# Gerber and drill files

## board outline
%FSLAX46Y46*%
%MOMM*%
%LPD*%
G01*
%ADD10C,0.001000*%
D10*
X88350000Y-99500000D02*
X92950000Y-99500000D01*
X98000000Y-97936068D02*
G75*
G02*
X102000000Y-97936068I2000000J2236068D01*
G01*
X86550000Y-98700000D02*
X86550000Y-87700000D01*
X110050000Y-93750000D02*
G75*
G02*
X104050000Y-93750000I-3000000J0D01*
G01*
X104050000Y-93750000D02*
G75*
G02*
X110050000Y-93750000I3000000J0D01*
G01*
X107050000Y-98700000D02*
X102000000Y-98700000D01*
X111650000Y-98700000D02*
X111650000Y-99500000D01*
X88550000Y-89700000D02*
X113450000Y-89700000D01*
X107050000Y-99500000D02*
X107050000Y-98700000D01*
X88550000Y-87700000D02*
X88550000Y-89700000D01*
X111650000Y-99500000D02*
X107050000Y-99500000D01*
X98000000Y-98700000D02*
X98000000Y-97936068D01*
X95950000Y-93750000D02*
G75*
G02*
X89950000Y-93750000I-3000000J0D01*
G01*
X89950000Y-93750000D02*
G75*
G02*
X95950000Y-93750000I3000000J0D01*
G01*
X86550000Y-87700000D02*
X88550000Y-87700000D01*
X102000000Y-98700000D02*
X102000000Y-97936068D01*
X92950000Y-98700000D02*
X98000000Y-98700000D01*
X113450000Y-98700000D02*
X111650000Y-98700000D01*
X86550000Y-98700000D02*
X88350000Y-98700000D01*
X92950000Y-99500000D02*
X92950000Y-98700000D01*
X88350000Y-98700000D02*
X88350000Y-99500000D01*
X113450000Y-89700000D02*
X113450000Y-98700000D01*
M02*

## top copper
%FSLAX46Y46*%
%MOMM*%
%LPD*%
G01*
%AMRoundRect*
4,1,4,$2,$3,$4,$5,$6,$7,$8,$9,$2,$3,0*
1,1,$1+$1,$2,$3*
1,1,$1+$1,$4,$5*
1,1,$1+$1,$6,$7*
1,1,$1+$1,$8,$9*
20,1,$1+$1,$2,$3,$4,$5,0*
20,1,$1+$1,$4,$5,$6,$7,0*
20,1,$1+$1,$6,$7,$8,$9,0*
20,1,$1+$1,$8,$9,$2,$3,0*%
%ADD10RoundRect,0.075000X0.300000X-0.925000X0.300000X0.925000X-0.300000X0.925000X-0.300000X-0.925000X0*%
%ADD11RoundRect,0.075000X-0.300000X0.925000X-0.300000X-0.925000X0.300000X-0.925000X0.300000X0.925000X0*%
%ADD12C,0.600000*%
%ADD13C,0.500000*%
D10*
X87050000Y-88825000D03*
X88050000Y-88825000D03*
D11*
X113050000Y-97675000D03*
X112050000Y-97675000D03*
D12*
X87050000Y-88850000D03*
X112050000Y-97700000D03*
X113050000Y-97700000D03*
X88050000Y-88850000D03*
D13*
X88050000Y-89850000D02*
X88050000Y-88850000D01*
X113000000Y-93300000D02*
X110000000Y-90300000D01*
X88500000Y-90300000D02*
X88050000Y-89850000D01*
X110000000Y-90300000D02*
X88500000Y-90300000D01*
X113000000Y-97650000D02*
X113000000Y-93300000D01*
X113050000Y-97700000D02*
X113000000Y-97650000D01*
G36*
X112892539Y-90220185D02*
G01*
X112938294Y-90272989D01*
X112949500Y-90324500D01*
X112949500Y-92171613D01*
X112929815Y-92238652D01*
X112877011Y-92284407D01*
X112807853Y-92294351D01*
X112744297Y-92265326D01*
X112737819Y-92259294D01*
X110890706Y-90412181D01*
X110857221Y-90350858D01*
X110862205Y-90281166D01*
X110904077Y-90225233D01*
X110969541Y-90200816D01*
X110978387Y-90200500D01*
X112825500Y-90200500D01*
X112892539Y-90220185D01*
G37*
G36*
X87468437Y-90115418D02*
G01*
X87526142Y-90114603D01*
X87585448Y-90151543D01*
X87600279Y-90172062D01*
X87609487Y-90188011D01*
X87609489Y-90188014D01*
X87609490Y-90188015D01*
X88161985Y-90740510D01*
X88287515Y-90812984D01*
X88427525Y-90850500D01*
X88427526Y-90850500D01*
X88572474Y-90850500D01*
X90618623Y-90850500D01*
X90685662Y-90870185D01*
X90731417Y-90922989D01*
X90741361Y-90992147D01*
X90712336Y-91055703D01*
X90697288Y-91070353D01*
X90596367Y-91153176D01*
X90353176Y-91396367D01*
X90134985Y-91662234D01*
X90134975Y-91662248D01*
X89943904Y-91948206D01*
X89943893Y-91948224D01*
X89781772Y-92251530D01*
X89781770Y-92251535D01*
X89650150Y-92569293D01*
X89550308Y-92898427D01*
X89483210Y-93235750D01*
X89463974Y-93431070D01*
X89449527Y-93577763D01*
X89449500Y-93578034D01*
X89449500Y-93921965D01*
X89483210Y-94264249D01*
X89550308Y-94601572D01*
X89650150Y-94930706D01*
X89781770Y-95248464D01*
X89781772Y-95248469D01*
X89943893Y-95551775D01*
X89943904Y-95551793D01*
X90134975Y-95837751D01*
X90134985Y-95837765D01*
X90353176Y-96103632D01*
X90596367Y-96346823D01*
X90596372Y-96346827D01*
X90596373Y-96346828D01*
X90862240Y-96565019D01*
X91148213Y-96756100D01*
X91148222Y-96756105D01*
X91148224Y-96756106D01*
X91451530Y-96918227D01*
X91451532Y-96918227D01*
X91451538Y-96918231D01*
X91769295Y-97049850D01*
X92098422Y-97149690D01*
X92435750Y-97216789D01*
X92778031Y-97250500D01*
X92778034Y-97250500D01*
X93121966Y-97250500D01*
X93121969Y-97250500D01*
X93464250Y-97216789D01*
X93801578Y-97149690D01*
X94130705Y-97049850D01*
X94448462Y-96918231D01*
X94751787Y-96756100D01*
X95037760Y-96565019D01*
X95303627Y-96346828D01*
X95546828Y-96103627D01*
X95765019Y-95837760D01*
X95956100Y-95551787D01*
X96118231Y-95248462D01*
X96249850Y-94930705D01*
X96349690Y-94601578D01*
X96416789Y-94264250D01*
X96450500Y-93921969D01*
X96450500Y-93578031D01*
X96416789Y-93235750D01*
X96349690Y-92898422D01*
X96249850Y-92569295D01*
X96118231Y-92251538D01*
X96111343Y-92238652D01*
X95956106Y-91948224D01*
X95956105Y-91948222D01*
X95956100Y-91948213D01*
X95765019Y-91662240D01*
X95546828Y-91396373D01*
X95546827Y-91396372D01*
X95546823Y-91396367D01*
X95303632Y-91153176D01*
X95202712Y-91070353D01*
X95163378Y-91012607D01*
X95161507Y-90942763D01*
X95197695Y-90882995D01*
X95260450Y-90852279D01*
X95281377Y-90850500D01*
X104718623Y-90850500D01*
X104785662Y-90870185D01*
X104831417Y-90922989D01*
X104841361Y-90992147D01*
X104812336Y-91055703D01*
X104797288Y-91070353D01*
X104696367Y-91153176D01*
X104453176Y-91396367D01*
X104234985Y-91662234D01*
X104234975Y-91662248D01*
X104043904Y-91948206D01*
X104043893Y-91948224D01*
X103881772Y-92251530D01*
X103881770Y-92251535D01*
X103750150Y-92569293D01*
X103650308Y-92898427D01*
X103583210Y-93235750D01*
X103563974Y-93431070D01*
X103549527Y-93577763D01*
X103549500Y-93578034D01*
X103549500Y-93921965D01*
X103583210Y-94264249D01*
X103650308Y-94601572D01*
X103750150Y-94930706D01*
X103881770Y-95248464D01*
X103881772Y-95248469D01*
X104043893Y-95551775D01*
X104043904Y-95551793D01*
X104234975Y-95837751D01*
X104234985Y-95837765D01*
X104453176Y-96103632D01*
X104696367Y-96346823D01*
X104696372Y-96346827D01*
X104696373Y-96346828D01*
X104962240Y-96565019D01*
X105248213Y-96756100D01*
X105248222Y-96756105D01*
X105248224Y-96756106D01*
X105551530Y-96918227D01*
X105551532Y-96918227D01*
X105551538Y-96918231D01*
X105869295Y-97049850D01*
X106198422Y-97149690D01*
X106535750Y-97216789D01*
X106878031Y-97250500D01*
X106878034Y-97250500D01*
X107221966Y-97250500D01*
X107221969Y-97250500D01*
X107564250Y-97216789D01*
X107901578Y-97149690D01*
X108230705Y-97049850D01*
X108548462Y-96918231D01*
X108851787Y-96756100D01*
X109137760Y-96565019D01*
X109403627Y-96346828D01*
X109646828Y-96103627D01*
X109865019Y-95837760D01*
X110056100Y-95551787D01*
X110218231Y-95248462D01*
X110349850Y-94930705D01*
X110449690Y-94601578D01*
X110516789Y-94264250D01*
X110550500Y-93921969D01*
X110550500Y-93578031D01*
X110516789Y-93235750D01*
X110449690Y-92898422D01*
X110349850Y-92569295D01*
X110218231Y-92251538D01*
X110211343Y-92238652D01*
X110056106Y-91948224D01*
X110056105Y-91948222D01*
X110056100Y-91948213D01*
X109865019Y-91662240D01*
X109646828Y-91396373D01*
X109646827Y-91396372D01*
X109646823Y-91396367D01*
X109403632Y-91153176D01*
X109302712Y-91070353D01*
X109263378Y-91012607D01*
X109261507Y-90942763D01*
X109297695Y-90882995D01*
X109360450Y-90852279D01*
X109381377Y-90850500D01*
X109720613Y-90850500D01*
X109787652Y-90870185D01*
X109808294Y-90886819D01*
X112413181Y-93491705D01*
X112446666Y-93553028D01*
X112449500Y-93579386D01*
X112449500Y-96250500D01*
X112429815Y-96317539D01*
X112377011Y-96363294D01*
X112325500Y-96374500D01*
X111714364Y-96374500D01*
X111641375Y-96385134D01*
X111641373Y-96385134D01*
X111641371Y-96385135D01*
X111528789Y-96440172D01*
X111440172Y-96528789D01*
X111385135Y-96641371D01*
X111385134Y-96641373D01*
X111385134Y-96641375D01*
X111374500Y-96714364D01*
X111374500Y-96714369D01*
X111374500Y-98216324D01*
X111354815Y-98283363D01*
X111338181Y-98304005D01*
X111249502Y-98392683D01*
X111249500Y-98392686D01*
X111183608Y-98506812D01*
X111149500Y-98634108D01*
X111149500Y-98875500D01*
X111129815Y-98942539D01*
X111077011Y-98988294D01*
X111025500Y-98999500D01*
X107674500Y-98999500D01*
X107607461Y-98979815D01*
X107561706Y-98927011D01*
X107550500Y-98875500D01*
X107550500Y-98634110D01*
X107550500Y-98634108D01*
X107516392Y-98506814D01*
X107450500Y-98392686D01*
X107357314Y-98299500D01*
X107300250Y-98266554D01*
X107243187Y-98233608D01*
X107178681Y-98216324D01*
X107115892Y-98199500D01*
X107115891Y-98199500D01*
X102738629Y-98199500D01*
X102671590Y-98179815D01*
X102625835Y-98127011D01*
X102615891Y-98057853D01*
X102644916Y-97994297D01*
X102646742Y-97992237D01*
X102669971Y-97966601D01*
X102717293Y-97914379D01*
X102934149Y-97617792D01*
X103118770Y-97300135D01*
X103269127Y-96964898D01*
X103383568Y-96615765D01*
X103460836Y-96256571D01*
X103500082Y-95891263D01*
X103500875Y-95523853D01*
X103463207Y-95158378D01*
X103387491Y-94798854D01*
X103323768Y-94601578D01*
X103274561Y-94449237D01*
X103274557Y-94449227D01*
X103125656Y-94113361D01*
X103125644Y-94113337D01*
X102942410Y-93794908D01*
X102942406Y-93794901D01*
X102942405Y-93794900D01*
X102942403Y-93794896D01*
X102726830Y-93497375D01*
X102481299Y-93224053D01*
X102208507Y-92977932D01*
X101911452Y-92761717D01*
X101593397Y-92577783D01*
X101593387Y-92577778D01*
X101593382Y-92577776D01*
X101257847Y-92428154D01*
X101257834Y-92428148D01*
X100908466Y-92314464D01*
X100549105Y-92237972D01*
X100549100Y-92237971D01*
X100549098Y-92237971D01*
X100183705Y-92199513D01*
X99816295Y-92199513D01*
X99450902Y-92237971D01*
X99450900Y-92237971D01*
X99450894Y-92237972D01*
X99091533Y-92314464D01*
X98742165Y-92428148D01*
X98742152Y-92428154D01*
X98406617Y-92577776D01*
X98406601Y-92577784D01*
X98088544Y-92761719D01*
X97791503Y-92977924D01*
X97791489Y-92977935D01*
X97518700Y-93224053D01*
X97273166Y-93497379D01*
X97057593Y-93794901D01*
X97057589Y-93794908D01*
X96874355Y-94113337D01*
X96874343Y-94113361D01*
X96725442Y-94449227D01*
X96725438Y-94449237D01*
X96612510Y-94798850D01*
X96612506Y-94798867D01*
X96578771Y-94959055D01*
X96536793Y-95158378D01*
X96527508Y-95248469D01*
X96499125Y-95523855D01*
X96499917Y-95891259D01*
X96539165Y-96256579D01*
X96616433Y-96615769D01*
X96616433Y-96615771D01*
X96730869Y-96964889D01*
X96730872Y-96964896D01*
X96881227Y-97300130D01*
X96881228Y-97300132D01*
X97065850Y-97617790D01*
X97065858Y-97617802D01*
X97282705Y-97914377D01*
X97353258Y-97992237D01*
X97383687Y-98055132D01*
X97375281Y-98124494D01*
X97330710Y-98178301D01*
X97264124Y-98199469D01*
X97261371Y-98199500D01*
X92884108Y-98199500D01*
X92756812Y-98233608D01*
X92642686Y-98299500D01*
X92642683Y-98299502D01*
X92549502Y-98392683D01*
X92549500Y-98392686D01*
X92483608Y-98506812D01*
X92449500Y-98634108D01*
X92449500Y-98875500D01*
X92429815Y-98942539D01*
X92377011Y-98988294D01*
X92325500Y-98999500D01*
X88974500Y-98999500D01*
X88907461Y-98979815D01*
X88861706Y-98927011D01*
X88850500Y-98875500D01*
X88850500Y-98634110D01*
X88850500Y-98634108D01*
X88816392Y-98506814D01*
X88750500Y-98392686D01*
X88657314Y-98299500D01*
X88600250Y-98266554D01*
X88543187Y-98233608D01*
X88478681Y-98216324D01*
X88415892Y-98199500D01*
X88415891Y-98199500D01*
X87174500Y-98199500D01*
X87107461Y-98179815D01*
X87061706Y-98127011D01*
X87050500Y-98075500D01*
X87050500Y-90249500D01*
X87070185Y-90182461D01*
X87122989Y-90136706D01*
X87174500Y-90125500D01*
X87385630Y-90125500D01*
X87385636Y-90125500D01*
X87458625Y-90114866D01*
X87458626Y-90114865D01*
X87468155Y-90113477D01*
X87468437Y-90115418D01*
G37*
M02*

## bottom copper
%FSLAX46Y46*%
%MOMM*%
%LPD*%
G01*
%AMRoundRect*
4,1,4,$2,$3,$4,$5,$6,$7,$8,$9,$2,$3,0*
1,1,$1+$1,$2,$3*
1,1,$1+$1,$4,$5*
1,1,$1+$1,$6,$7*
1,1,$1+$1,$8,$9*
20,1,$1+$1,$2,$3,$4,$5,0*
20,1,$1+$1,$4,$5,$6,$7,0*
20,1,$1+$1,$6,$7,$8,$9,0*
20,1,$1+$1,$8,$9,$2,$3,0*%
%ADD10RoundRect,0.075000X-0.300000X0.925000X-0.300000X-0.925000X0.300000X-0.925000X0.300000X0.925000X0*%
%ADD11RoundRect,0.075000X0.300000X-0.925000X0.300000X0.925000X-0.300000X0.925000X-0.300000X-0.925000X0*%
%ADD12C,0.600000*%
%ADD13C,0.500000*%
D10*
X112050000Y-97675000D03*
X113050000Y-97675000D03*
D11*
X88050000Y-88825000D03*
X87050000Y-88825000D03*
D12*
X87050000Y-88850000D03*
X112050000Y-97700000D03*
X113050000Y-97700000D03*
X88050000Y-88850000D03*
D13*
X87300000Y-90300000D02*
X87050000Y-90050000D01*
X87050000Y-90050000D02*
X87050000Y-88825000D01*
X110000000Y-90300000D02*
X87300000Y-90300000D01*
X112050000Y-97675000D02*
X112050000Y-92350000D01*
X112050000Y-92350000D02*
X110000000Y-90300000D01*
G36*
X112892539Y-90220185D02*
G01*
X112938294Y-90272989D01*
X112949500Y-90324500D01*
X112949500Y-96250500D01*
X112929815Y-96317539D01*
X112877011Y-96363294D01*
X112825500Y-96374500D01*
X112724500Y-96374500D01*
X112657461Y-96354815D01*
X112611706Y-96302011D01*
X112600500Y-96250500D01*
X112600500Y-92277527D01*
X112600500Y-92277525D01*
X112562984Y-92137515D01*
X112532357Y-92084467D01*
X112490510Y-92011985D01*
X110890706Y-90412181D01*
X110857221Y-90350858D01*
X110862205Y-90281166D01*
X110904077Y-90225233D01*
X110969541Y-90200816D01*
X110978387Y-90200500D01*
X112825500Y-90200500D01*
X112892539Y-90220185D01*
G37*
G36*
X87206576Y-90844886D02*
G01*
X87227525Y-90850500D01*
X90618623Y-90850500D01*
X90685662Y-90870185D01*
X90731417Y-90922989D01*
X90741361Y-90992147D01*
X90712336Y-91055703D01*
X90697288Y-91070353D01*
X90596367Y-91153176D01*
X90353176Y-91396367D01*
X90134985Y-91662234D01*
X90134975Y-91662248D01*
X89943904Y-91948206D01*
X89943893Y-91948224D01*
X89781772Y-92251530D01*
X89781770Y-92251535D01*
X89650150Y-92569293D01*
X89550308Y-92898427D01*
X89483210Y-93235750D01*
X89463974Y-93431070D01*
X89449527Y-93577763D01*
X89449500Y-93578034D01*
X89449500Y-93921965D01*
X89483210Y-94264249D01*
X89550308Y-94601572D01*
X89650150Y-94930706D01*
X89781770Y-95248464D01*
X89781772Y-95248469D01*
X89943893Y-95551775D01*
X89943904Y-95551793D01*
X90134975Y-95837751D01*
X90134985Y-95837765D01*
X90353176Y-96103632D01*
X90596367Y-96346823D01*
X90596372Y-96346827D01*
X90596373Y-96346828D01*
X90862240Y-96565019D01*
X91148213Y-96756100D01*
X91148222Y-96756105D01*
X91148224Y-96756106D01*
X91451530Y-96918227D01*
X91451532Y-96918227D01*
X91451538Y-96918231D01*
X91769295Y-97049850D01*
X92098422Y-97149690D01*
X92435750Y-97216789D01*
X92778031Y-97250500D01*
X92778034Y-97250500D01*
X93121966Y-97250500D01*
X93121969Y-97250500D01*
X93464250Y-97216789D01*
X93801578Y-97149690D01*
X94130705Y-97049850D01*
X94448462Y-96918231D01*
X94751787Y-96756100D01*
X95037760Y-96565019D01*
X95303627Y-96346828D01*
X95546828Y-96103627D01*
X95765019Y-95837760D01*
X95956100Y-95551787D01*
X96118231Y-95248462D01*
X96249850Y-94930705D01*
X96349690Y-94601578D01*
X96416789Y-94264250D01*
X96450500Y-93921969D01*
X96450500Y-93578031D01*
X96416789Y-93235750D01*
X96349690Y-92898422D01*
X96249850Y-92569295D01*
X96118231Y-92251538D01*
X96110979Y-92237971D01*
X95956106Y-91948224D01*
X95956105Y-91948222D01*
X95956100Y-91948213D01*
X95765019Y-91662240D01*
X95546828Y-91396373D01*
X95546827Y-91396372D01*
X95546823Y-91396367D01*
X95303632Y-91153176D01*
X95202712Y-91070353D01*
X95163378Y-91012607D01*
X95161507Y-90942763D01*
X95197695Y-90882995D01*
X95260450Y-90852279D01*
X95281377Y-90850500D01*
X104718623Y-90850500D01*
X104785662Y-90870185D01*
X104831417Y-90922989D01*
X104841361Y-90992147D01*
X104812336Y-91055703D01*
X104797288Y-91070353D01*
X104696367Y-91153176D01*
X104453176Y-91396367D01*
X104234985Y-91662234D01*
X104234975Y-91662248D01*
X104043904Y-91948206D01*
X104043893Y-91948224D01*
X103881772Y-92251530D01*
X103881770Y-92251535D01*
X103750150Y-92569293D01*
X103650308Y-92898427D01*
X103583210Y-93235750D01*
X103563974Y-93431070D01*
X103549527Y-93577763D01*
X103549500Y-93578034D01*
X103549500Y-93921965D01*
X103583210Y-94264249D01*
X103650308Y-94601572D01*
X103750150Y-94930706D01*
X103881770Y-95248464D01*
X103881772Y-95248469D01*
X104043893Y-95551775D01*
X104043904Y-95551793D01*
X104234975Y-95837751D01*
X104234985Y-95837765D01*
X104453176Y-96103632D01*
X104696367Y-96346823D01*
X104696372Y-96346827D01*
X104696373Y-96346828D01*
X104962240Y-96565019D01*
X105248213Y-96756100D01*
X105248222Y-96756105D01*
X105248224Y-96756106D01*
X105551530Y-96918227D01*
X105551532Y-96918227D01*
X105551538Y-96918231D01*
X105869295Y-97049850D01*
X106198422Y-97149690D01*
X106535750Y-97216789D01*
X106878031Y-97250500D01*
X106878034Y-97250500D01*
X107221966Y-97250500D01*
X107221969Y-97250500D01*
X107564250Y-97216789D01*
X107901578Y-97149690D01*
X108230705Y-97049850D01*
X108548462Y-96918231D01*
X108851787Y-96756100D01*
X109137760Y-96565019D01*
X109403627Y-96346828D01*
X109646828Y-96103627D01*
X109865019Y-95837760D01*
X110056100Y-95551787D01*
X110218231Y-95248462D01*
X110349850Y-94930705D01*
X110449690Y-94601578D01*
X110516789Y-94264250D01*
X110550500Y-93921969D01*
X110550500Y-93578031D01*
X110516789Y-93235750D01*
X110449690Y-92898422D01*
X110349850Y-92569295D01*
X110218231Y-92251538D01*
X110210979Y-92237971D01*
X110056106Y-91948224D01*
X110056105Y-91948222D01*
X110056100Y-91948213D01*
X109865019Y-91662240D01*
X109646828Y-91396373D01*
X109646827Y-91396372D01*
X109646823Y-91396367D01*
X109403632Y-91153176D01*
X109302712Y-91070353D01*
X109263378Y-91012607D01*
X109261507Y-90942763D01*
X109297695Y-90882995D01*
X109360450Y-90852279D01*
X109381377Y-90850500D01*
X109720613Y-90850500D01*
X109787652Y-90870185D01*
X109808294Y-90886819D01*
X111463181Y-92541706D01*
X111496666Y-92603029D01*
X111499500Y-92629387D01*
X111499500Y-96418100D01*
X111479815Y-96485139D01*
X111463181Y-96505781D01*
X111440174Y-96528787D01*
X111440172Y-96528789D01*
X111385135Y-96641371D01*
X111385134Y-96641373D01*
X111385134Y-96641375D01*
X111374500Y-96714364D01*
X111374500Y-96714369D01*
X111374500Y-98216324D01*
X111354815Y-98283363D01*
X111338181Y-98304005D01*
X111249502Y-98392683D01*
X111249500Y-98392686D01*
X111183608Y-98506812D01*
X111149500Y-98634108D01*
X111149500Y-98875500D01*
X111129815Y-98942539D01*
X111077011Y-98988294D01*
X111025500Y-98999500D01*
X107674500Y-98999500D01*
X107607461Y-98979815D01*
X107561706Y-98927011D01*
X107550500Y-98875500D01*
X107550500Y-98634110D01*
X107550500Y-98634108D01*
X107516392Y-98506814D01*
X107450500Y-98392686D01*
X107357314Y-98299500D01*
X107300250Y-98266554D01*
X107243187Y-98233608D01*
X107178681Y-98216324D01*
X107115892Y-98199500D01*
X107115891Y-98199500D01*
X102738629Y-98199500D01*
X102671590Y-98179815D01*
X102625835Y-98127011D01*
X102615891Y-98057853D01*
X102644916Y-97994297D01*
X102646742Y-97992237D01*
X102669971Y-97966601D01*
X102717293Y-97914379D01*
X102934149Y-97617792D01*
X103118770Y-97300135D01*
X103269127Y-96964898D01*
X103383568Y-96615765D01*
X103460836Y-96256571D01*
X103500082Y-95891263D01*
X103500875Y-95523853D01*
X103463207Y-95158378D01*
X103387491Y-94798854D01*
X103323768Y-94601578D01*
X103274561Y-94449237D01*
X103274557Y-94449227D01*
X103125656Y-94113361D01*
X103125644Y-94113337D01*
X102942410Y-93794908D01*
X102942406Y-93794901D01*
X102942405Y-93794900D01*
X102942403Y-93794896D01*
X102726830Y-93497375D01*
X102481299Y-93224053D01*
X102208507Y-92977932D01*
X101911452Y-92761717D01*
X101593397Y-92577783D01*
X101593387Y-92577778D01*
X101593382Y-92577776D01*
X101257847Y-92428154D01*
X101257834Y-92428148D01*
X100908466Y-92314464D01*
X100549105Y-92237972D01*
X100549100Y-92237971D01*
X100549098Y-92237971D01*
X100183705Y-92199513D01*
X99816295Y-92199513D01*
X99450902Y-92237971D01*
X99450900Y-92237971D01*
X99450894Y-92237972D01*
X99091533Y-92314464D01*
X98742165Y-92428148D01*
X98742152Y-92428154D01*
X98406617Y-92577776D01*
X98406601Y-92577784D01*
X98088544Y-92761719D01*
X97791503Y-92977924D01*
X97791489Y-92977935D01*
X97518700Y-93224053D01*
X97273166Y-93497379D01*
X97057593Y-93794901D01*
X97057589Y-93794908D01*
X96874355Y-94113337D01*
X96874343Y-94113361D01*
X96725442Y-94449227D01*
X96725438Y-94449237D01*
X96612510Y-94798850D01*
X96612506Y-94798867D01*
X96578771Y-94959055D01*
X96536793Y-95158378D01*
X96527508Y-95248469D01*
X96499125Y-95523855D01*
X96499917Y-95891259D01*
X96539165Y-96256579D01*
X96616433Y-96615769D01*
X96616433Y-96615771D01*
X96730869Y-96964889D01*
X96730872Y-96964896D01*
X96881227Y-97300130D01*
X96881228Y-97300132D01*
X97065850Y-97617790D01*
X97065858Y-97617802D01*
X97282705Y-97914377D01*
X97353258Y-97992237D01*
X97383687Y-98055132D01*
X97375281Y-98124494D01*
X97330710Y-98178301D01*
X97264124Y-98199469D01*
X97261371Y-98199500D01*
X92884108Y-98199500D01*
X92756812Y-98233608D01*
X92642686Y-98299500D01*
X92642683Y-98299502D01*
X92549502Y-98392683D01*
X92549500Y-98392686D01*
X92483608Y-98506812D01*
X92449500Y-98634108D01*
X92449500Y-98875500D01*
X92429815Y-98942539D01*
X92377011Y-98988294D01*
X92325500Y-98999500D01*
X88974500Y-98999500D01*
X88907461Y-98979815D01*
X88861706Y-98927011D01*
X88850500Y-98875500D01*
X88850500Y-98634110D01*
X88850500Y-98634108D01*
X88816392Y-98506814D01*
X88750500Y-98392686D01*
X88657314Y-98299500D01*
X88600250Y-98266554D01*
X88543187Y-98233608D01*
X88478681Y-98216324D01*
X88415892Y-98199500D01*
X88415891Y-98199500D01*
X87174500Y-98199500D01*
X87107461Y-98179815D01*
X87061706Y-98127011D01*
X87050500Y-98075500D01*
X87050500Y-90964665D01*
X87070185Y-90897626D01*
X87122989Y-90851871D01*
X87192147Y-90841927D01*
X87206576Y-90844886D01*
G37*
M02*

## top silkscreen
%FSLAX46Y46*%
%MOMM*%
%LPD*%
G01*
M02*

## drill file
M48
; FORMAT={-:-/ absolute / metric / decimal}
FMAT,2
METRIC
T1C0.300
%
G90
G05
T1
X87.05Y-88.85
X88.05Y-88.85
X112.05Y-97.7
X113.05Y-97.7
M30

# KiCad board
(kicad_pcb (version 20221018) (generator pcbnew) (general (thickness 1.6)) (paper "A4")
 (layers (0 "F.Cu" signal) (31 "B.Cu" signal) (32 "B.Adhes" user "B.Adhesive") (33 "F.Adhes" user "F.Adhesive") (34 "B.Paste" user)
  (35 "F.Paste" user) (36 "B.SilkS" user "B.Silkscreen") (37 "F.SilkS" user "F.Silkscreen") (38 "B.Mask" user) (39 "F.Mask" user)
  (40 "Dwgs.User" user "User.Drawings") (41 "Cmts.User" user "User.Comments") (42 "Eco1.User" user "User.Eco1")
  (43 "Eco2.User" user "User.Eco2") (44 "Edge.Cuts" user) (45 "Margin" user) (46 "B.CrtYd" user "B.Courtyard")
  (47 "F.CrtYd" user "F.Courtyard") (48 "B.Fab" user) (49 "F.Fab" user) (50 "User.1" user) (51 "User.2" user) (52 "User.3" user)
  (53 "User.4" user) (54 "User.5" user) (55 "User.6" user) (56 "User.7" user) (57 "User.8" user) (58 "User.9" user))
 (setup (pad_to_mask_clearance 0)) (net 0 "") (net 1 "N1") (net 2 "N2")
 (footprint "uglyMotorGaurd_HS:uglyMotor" (layer "F.Cu") (at 87.55 89.825)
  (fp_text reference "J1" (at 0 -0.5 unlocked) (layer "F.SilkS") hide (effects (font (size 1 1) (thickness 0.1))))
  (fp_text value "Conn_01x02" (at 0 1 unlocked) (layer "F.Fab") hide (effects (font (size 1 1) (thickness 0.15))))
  (pad "1" smd roundrect (at -0.5 -1 90) (size 2 0.75) (layers "F.Cu" "F.Paste" "F.Mask") (roundrect_rratio 0.1) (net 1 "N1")
   (thermal_bridge_angle 45))
  (pad "2" smd roundrect (at 0.5 -1 90) (size 2 0.75) (layers "F.Cu" "F.Paste" "F.Mask") (roundrect_rratio 0.1) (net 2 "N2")
   (thermal_bridge_angle 45)))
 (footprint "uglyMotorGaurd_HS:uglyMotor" (layer "F.Cu") (at 112.55 96.675 180)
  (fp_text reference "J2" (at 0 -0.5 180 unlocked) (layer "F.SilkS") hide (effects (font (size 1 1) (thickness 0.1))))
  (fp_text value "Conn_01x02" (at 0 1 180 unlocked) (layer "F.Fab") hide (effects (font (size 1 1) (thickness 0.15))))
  (pad "1" smd roundrect (at -0.5 -1 270) (size 2 0.75) (layers "F.Cu" "F.Paste" "F.Mask") (roundrect_rratio 0.1) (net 2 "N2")
   (thermal_bridge_angle 45))
  (pad "2" smd roundrect (at 0.5 -1 270) (size 2 0.75) (layers "F.Cu" "F.Paste" "F.Mask") (roundrect_rratio 0.1) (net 1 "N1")
   (thermal_bridge_angle 45)))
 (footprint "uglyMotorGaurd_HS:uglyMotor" (layer "B.Cu") (at 112.55 96.675)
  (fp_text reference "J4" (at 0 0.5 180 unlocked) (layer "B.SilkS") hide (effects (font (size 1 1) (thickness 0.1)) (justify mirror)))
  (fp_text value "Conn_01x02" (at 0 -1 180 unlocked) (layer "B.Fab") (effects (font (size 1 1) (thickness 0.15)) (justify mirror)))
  (pad "1" smd roundrect (at -0.5 1 270) (size 2 0.75) (layers "B.Cu" "B.Paste" "B.Mask") (roundrect_rratio 0.1) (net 1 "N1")
   (thermal_bridge_angle 45))
  (pad "2" smd roundrect (at 0.5 1 270) (size 2 0.75) (layers "B.Cu" "B.Paste" "B.Mask") (roundrect_rratio 0.1) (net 2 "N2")
   (thermal_bridge_angle 45)))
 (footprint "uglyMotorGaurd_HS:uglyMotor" (layer "B.Cu") (at 87.55 89.825 180)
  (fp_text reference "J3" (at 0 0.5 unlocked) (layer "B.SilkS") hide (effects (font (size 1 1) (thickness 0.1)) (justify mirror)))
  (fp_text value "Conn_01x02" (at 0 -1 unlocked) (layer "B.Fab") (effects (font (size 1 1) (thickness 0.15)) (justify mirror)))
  (pad "1" smd roundrect (at -0.5 1 90) (size 2 0.75) (layers "B.Cu" "B.Paste" "B.Mask") (roundrect_rratio 0.1) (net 2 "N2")
   (thermal_bridge_angle 45))
  (pad "2" smd roundrect (at 0.5 1 90) (size 2 0.75) (layers "B.Cu" "B.Paste" "B.Mask") (roundrect_rratio 0.1) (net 1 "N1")
   (thermal_bridge_angle 45)))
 (gr_line (start 88.35 99.5) (end 92.95 99.5) (stroke (width 0.001) (type solid)) (layer "Edge.Cuts"))
 (gr_arc (start 98 97.936068) (mid 100 92.7) (end 102 97.936068) (stroke (width 0.001) (type solid)) (layer "Edge.Cuts"))
 (gr_line (start 86.55 98.7) (end 86.55 87.7) (stroke (width 0.001) (type solid)) (layer "Edge.Cuts"))
 (gr_circle (center 107.05 93.75) (end 110.05 93.75) (stroke (width 0.001) (type solid)) (fill none) (layer "Edge.Cuts"))
 (gr_line (start 107.05 98.7) (end 102 98.7) (stroke (width 0.001) (type solid)) (layer "Edge.Cuts"))
 (gr_line (start 111.65 98.7) (end 111.65 99.5) (stroke (width 0.001) (type solid)) (layer "Edge.Cuts"))
 (gr_line (start 88.55 89.7) (end 113.45 89.7) (stroke (width 0.001) (type solid)) (layer "Edge.Cuts"))
 (gr_line (start 107.05 99.5) (end 107.05 98.7) (stroke (width 0.001) (type solid)) (layer "Edge.Cuts"))
 (gr_line (start 88.55 87.7) (end 88.55 89.7) (stroke (width 0.001) (type solid)) (layer "Edge.Cuts"))
 (gr_line (start 111.65 99.5) (end 107.05 99.5) (stroke (width 0.001) (type solid)) (layer "Edge.Cuts"))
 (gr_line (start 98 98.7) (end 98 97.936068) (stroke (width 0.001) (type solid)) (layer "Edge.Cuts"))
 (gr_circle (center 92.95 93.75) (end 95.95 93.75) (stroke (width 0.001) (type solid)) (fill none) (layer "Edge.Cuts"))
 (gr_line (start 86.55 87.7) (end 88.55 87.7) (stroke (width 0.001) (type solid)) (layer "Edge.Cuts"))
 (gr_line (start 102 98.7) (end 102 97.936068) (stroke (width 0.001) (type solid)) (layer "Edge.Cuts"))
 (gr_line (start 92.95 98.7) (end 98 98.7) (stroke (width 0.001) (type solid)) (layer "Edge.Cuts"))
 (gr_line (start 113.45 98.7) (end 111.65 98.7) (stroke (width 0.001) (type solid)) (layer "Edge.Cuts"))
 (gr_line (start 86.55 98.7) (end 88.35 98.7) (stroke (width 0.001) (type solid)) (layer "Edge.Cuts"))
 (gr_line (start 92.95 99.5) (end 92.95 98.7) (stroke (width 0.001) (type solid)) (layer "Edge.Cuts"))
 (gr_line (start 88.35 98.7) (end 88.35 99.5) (stroke (width 0.001) (type solid)) (layer "Edge.Cuts"))
 (gr_line (start 113.45 89.7) (end 113.45 98.7) (stroke (width 0.001) (type solid)) (layer "Edge.Cuts"))
 (via (at 87.05 88.85) (size 0.6) (drill 0.3) (layers "F.Cu" "B.Cu") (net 1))
 (via (at 112.05 97.7) (size 0.6) (drill 0.3) (layers "F.Cu" "B.Cu") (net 1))
 (segment (start 87.3 90.3) (end 87.05 90.05) (width 0.5) (layer "B.Cu") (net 1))
 (segment (start 87.05 90.05) (end 87.05 88.825) (width 0.5) (layer "B.Cu") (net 1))
 (segment (start 110 90.3) (end 87.3 90.3) (width 0.5) (layer "B.Cu") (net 1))
 (segment (start 112.05 97.675) (end 112.05 92.35) (width 0.5) (layer "B.Cu") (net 1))
 (segment (start 112.05 92.35) (end 110 90.3) (width 0.5) (layer "B.Cu") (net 1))
 (segment (start 88.05 89.85) (end 88.05 88.85) (width 0.5) (layer "F.Cu") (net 2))
 (segment (start 113 93.3) (end 110 90.3) (width 0.5) (layer "F.Cu") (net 2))
 (segment (start 88.5 90.3) (end 88.05 89.85) (width 0.5) (layer "F.Cu") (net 2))
 (segment (start 110 90.3) (end 88.5 90.3) (width 0.5) (layer "F.Cu") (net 2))
 (segment (start 113 97.65) (end 113 93.3) (width 0.5) (layer "F.Cu") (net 2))
 (segment (start 113.05 97.7) (end 113 97.65) (width 0.5) (layer "F.Cu") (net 2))
 (via (at 113.05 97.7) (size 0.6) (drill 0.3) (layers "F.Cu" "B.Cu") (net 2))
 (via (at 88.05 88.85) (size 0.6) (drill 0.3) (layers "F.Cu" "B.Cu") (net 2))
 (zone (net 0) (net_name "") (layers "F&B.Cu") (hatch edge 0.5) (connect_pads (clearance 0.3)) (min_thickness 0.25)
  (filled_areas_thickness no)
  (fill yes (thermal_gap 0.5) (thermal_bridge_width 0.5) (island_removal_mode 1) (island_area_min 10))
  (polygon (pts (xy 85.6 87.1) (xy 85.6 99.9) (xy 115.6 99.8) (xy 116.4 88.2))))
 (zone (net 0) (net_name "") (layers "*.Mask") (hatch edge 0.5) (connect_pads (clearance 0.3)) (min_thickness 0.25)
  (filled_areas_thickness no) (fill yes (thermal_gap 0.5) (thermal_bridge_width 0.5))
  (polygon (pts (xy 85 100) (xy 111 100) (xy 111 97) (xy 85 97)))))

